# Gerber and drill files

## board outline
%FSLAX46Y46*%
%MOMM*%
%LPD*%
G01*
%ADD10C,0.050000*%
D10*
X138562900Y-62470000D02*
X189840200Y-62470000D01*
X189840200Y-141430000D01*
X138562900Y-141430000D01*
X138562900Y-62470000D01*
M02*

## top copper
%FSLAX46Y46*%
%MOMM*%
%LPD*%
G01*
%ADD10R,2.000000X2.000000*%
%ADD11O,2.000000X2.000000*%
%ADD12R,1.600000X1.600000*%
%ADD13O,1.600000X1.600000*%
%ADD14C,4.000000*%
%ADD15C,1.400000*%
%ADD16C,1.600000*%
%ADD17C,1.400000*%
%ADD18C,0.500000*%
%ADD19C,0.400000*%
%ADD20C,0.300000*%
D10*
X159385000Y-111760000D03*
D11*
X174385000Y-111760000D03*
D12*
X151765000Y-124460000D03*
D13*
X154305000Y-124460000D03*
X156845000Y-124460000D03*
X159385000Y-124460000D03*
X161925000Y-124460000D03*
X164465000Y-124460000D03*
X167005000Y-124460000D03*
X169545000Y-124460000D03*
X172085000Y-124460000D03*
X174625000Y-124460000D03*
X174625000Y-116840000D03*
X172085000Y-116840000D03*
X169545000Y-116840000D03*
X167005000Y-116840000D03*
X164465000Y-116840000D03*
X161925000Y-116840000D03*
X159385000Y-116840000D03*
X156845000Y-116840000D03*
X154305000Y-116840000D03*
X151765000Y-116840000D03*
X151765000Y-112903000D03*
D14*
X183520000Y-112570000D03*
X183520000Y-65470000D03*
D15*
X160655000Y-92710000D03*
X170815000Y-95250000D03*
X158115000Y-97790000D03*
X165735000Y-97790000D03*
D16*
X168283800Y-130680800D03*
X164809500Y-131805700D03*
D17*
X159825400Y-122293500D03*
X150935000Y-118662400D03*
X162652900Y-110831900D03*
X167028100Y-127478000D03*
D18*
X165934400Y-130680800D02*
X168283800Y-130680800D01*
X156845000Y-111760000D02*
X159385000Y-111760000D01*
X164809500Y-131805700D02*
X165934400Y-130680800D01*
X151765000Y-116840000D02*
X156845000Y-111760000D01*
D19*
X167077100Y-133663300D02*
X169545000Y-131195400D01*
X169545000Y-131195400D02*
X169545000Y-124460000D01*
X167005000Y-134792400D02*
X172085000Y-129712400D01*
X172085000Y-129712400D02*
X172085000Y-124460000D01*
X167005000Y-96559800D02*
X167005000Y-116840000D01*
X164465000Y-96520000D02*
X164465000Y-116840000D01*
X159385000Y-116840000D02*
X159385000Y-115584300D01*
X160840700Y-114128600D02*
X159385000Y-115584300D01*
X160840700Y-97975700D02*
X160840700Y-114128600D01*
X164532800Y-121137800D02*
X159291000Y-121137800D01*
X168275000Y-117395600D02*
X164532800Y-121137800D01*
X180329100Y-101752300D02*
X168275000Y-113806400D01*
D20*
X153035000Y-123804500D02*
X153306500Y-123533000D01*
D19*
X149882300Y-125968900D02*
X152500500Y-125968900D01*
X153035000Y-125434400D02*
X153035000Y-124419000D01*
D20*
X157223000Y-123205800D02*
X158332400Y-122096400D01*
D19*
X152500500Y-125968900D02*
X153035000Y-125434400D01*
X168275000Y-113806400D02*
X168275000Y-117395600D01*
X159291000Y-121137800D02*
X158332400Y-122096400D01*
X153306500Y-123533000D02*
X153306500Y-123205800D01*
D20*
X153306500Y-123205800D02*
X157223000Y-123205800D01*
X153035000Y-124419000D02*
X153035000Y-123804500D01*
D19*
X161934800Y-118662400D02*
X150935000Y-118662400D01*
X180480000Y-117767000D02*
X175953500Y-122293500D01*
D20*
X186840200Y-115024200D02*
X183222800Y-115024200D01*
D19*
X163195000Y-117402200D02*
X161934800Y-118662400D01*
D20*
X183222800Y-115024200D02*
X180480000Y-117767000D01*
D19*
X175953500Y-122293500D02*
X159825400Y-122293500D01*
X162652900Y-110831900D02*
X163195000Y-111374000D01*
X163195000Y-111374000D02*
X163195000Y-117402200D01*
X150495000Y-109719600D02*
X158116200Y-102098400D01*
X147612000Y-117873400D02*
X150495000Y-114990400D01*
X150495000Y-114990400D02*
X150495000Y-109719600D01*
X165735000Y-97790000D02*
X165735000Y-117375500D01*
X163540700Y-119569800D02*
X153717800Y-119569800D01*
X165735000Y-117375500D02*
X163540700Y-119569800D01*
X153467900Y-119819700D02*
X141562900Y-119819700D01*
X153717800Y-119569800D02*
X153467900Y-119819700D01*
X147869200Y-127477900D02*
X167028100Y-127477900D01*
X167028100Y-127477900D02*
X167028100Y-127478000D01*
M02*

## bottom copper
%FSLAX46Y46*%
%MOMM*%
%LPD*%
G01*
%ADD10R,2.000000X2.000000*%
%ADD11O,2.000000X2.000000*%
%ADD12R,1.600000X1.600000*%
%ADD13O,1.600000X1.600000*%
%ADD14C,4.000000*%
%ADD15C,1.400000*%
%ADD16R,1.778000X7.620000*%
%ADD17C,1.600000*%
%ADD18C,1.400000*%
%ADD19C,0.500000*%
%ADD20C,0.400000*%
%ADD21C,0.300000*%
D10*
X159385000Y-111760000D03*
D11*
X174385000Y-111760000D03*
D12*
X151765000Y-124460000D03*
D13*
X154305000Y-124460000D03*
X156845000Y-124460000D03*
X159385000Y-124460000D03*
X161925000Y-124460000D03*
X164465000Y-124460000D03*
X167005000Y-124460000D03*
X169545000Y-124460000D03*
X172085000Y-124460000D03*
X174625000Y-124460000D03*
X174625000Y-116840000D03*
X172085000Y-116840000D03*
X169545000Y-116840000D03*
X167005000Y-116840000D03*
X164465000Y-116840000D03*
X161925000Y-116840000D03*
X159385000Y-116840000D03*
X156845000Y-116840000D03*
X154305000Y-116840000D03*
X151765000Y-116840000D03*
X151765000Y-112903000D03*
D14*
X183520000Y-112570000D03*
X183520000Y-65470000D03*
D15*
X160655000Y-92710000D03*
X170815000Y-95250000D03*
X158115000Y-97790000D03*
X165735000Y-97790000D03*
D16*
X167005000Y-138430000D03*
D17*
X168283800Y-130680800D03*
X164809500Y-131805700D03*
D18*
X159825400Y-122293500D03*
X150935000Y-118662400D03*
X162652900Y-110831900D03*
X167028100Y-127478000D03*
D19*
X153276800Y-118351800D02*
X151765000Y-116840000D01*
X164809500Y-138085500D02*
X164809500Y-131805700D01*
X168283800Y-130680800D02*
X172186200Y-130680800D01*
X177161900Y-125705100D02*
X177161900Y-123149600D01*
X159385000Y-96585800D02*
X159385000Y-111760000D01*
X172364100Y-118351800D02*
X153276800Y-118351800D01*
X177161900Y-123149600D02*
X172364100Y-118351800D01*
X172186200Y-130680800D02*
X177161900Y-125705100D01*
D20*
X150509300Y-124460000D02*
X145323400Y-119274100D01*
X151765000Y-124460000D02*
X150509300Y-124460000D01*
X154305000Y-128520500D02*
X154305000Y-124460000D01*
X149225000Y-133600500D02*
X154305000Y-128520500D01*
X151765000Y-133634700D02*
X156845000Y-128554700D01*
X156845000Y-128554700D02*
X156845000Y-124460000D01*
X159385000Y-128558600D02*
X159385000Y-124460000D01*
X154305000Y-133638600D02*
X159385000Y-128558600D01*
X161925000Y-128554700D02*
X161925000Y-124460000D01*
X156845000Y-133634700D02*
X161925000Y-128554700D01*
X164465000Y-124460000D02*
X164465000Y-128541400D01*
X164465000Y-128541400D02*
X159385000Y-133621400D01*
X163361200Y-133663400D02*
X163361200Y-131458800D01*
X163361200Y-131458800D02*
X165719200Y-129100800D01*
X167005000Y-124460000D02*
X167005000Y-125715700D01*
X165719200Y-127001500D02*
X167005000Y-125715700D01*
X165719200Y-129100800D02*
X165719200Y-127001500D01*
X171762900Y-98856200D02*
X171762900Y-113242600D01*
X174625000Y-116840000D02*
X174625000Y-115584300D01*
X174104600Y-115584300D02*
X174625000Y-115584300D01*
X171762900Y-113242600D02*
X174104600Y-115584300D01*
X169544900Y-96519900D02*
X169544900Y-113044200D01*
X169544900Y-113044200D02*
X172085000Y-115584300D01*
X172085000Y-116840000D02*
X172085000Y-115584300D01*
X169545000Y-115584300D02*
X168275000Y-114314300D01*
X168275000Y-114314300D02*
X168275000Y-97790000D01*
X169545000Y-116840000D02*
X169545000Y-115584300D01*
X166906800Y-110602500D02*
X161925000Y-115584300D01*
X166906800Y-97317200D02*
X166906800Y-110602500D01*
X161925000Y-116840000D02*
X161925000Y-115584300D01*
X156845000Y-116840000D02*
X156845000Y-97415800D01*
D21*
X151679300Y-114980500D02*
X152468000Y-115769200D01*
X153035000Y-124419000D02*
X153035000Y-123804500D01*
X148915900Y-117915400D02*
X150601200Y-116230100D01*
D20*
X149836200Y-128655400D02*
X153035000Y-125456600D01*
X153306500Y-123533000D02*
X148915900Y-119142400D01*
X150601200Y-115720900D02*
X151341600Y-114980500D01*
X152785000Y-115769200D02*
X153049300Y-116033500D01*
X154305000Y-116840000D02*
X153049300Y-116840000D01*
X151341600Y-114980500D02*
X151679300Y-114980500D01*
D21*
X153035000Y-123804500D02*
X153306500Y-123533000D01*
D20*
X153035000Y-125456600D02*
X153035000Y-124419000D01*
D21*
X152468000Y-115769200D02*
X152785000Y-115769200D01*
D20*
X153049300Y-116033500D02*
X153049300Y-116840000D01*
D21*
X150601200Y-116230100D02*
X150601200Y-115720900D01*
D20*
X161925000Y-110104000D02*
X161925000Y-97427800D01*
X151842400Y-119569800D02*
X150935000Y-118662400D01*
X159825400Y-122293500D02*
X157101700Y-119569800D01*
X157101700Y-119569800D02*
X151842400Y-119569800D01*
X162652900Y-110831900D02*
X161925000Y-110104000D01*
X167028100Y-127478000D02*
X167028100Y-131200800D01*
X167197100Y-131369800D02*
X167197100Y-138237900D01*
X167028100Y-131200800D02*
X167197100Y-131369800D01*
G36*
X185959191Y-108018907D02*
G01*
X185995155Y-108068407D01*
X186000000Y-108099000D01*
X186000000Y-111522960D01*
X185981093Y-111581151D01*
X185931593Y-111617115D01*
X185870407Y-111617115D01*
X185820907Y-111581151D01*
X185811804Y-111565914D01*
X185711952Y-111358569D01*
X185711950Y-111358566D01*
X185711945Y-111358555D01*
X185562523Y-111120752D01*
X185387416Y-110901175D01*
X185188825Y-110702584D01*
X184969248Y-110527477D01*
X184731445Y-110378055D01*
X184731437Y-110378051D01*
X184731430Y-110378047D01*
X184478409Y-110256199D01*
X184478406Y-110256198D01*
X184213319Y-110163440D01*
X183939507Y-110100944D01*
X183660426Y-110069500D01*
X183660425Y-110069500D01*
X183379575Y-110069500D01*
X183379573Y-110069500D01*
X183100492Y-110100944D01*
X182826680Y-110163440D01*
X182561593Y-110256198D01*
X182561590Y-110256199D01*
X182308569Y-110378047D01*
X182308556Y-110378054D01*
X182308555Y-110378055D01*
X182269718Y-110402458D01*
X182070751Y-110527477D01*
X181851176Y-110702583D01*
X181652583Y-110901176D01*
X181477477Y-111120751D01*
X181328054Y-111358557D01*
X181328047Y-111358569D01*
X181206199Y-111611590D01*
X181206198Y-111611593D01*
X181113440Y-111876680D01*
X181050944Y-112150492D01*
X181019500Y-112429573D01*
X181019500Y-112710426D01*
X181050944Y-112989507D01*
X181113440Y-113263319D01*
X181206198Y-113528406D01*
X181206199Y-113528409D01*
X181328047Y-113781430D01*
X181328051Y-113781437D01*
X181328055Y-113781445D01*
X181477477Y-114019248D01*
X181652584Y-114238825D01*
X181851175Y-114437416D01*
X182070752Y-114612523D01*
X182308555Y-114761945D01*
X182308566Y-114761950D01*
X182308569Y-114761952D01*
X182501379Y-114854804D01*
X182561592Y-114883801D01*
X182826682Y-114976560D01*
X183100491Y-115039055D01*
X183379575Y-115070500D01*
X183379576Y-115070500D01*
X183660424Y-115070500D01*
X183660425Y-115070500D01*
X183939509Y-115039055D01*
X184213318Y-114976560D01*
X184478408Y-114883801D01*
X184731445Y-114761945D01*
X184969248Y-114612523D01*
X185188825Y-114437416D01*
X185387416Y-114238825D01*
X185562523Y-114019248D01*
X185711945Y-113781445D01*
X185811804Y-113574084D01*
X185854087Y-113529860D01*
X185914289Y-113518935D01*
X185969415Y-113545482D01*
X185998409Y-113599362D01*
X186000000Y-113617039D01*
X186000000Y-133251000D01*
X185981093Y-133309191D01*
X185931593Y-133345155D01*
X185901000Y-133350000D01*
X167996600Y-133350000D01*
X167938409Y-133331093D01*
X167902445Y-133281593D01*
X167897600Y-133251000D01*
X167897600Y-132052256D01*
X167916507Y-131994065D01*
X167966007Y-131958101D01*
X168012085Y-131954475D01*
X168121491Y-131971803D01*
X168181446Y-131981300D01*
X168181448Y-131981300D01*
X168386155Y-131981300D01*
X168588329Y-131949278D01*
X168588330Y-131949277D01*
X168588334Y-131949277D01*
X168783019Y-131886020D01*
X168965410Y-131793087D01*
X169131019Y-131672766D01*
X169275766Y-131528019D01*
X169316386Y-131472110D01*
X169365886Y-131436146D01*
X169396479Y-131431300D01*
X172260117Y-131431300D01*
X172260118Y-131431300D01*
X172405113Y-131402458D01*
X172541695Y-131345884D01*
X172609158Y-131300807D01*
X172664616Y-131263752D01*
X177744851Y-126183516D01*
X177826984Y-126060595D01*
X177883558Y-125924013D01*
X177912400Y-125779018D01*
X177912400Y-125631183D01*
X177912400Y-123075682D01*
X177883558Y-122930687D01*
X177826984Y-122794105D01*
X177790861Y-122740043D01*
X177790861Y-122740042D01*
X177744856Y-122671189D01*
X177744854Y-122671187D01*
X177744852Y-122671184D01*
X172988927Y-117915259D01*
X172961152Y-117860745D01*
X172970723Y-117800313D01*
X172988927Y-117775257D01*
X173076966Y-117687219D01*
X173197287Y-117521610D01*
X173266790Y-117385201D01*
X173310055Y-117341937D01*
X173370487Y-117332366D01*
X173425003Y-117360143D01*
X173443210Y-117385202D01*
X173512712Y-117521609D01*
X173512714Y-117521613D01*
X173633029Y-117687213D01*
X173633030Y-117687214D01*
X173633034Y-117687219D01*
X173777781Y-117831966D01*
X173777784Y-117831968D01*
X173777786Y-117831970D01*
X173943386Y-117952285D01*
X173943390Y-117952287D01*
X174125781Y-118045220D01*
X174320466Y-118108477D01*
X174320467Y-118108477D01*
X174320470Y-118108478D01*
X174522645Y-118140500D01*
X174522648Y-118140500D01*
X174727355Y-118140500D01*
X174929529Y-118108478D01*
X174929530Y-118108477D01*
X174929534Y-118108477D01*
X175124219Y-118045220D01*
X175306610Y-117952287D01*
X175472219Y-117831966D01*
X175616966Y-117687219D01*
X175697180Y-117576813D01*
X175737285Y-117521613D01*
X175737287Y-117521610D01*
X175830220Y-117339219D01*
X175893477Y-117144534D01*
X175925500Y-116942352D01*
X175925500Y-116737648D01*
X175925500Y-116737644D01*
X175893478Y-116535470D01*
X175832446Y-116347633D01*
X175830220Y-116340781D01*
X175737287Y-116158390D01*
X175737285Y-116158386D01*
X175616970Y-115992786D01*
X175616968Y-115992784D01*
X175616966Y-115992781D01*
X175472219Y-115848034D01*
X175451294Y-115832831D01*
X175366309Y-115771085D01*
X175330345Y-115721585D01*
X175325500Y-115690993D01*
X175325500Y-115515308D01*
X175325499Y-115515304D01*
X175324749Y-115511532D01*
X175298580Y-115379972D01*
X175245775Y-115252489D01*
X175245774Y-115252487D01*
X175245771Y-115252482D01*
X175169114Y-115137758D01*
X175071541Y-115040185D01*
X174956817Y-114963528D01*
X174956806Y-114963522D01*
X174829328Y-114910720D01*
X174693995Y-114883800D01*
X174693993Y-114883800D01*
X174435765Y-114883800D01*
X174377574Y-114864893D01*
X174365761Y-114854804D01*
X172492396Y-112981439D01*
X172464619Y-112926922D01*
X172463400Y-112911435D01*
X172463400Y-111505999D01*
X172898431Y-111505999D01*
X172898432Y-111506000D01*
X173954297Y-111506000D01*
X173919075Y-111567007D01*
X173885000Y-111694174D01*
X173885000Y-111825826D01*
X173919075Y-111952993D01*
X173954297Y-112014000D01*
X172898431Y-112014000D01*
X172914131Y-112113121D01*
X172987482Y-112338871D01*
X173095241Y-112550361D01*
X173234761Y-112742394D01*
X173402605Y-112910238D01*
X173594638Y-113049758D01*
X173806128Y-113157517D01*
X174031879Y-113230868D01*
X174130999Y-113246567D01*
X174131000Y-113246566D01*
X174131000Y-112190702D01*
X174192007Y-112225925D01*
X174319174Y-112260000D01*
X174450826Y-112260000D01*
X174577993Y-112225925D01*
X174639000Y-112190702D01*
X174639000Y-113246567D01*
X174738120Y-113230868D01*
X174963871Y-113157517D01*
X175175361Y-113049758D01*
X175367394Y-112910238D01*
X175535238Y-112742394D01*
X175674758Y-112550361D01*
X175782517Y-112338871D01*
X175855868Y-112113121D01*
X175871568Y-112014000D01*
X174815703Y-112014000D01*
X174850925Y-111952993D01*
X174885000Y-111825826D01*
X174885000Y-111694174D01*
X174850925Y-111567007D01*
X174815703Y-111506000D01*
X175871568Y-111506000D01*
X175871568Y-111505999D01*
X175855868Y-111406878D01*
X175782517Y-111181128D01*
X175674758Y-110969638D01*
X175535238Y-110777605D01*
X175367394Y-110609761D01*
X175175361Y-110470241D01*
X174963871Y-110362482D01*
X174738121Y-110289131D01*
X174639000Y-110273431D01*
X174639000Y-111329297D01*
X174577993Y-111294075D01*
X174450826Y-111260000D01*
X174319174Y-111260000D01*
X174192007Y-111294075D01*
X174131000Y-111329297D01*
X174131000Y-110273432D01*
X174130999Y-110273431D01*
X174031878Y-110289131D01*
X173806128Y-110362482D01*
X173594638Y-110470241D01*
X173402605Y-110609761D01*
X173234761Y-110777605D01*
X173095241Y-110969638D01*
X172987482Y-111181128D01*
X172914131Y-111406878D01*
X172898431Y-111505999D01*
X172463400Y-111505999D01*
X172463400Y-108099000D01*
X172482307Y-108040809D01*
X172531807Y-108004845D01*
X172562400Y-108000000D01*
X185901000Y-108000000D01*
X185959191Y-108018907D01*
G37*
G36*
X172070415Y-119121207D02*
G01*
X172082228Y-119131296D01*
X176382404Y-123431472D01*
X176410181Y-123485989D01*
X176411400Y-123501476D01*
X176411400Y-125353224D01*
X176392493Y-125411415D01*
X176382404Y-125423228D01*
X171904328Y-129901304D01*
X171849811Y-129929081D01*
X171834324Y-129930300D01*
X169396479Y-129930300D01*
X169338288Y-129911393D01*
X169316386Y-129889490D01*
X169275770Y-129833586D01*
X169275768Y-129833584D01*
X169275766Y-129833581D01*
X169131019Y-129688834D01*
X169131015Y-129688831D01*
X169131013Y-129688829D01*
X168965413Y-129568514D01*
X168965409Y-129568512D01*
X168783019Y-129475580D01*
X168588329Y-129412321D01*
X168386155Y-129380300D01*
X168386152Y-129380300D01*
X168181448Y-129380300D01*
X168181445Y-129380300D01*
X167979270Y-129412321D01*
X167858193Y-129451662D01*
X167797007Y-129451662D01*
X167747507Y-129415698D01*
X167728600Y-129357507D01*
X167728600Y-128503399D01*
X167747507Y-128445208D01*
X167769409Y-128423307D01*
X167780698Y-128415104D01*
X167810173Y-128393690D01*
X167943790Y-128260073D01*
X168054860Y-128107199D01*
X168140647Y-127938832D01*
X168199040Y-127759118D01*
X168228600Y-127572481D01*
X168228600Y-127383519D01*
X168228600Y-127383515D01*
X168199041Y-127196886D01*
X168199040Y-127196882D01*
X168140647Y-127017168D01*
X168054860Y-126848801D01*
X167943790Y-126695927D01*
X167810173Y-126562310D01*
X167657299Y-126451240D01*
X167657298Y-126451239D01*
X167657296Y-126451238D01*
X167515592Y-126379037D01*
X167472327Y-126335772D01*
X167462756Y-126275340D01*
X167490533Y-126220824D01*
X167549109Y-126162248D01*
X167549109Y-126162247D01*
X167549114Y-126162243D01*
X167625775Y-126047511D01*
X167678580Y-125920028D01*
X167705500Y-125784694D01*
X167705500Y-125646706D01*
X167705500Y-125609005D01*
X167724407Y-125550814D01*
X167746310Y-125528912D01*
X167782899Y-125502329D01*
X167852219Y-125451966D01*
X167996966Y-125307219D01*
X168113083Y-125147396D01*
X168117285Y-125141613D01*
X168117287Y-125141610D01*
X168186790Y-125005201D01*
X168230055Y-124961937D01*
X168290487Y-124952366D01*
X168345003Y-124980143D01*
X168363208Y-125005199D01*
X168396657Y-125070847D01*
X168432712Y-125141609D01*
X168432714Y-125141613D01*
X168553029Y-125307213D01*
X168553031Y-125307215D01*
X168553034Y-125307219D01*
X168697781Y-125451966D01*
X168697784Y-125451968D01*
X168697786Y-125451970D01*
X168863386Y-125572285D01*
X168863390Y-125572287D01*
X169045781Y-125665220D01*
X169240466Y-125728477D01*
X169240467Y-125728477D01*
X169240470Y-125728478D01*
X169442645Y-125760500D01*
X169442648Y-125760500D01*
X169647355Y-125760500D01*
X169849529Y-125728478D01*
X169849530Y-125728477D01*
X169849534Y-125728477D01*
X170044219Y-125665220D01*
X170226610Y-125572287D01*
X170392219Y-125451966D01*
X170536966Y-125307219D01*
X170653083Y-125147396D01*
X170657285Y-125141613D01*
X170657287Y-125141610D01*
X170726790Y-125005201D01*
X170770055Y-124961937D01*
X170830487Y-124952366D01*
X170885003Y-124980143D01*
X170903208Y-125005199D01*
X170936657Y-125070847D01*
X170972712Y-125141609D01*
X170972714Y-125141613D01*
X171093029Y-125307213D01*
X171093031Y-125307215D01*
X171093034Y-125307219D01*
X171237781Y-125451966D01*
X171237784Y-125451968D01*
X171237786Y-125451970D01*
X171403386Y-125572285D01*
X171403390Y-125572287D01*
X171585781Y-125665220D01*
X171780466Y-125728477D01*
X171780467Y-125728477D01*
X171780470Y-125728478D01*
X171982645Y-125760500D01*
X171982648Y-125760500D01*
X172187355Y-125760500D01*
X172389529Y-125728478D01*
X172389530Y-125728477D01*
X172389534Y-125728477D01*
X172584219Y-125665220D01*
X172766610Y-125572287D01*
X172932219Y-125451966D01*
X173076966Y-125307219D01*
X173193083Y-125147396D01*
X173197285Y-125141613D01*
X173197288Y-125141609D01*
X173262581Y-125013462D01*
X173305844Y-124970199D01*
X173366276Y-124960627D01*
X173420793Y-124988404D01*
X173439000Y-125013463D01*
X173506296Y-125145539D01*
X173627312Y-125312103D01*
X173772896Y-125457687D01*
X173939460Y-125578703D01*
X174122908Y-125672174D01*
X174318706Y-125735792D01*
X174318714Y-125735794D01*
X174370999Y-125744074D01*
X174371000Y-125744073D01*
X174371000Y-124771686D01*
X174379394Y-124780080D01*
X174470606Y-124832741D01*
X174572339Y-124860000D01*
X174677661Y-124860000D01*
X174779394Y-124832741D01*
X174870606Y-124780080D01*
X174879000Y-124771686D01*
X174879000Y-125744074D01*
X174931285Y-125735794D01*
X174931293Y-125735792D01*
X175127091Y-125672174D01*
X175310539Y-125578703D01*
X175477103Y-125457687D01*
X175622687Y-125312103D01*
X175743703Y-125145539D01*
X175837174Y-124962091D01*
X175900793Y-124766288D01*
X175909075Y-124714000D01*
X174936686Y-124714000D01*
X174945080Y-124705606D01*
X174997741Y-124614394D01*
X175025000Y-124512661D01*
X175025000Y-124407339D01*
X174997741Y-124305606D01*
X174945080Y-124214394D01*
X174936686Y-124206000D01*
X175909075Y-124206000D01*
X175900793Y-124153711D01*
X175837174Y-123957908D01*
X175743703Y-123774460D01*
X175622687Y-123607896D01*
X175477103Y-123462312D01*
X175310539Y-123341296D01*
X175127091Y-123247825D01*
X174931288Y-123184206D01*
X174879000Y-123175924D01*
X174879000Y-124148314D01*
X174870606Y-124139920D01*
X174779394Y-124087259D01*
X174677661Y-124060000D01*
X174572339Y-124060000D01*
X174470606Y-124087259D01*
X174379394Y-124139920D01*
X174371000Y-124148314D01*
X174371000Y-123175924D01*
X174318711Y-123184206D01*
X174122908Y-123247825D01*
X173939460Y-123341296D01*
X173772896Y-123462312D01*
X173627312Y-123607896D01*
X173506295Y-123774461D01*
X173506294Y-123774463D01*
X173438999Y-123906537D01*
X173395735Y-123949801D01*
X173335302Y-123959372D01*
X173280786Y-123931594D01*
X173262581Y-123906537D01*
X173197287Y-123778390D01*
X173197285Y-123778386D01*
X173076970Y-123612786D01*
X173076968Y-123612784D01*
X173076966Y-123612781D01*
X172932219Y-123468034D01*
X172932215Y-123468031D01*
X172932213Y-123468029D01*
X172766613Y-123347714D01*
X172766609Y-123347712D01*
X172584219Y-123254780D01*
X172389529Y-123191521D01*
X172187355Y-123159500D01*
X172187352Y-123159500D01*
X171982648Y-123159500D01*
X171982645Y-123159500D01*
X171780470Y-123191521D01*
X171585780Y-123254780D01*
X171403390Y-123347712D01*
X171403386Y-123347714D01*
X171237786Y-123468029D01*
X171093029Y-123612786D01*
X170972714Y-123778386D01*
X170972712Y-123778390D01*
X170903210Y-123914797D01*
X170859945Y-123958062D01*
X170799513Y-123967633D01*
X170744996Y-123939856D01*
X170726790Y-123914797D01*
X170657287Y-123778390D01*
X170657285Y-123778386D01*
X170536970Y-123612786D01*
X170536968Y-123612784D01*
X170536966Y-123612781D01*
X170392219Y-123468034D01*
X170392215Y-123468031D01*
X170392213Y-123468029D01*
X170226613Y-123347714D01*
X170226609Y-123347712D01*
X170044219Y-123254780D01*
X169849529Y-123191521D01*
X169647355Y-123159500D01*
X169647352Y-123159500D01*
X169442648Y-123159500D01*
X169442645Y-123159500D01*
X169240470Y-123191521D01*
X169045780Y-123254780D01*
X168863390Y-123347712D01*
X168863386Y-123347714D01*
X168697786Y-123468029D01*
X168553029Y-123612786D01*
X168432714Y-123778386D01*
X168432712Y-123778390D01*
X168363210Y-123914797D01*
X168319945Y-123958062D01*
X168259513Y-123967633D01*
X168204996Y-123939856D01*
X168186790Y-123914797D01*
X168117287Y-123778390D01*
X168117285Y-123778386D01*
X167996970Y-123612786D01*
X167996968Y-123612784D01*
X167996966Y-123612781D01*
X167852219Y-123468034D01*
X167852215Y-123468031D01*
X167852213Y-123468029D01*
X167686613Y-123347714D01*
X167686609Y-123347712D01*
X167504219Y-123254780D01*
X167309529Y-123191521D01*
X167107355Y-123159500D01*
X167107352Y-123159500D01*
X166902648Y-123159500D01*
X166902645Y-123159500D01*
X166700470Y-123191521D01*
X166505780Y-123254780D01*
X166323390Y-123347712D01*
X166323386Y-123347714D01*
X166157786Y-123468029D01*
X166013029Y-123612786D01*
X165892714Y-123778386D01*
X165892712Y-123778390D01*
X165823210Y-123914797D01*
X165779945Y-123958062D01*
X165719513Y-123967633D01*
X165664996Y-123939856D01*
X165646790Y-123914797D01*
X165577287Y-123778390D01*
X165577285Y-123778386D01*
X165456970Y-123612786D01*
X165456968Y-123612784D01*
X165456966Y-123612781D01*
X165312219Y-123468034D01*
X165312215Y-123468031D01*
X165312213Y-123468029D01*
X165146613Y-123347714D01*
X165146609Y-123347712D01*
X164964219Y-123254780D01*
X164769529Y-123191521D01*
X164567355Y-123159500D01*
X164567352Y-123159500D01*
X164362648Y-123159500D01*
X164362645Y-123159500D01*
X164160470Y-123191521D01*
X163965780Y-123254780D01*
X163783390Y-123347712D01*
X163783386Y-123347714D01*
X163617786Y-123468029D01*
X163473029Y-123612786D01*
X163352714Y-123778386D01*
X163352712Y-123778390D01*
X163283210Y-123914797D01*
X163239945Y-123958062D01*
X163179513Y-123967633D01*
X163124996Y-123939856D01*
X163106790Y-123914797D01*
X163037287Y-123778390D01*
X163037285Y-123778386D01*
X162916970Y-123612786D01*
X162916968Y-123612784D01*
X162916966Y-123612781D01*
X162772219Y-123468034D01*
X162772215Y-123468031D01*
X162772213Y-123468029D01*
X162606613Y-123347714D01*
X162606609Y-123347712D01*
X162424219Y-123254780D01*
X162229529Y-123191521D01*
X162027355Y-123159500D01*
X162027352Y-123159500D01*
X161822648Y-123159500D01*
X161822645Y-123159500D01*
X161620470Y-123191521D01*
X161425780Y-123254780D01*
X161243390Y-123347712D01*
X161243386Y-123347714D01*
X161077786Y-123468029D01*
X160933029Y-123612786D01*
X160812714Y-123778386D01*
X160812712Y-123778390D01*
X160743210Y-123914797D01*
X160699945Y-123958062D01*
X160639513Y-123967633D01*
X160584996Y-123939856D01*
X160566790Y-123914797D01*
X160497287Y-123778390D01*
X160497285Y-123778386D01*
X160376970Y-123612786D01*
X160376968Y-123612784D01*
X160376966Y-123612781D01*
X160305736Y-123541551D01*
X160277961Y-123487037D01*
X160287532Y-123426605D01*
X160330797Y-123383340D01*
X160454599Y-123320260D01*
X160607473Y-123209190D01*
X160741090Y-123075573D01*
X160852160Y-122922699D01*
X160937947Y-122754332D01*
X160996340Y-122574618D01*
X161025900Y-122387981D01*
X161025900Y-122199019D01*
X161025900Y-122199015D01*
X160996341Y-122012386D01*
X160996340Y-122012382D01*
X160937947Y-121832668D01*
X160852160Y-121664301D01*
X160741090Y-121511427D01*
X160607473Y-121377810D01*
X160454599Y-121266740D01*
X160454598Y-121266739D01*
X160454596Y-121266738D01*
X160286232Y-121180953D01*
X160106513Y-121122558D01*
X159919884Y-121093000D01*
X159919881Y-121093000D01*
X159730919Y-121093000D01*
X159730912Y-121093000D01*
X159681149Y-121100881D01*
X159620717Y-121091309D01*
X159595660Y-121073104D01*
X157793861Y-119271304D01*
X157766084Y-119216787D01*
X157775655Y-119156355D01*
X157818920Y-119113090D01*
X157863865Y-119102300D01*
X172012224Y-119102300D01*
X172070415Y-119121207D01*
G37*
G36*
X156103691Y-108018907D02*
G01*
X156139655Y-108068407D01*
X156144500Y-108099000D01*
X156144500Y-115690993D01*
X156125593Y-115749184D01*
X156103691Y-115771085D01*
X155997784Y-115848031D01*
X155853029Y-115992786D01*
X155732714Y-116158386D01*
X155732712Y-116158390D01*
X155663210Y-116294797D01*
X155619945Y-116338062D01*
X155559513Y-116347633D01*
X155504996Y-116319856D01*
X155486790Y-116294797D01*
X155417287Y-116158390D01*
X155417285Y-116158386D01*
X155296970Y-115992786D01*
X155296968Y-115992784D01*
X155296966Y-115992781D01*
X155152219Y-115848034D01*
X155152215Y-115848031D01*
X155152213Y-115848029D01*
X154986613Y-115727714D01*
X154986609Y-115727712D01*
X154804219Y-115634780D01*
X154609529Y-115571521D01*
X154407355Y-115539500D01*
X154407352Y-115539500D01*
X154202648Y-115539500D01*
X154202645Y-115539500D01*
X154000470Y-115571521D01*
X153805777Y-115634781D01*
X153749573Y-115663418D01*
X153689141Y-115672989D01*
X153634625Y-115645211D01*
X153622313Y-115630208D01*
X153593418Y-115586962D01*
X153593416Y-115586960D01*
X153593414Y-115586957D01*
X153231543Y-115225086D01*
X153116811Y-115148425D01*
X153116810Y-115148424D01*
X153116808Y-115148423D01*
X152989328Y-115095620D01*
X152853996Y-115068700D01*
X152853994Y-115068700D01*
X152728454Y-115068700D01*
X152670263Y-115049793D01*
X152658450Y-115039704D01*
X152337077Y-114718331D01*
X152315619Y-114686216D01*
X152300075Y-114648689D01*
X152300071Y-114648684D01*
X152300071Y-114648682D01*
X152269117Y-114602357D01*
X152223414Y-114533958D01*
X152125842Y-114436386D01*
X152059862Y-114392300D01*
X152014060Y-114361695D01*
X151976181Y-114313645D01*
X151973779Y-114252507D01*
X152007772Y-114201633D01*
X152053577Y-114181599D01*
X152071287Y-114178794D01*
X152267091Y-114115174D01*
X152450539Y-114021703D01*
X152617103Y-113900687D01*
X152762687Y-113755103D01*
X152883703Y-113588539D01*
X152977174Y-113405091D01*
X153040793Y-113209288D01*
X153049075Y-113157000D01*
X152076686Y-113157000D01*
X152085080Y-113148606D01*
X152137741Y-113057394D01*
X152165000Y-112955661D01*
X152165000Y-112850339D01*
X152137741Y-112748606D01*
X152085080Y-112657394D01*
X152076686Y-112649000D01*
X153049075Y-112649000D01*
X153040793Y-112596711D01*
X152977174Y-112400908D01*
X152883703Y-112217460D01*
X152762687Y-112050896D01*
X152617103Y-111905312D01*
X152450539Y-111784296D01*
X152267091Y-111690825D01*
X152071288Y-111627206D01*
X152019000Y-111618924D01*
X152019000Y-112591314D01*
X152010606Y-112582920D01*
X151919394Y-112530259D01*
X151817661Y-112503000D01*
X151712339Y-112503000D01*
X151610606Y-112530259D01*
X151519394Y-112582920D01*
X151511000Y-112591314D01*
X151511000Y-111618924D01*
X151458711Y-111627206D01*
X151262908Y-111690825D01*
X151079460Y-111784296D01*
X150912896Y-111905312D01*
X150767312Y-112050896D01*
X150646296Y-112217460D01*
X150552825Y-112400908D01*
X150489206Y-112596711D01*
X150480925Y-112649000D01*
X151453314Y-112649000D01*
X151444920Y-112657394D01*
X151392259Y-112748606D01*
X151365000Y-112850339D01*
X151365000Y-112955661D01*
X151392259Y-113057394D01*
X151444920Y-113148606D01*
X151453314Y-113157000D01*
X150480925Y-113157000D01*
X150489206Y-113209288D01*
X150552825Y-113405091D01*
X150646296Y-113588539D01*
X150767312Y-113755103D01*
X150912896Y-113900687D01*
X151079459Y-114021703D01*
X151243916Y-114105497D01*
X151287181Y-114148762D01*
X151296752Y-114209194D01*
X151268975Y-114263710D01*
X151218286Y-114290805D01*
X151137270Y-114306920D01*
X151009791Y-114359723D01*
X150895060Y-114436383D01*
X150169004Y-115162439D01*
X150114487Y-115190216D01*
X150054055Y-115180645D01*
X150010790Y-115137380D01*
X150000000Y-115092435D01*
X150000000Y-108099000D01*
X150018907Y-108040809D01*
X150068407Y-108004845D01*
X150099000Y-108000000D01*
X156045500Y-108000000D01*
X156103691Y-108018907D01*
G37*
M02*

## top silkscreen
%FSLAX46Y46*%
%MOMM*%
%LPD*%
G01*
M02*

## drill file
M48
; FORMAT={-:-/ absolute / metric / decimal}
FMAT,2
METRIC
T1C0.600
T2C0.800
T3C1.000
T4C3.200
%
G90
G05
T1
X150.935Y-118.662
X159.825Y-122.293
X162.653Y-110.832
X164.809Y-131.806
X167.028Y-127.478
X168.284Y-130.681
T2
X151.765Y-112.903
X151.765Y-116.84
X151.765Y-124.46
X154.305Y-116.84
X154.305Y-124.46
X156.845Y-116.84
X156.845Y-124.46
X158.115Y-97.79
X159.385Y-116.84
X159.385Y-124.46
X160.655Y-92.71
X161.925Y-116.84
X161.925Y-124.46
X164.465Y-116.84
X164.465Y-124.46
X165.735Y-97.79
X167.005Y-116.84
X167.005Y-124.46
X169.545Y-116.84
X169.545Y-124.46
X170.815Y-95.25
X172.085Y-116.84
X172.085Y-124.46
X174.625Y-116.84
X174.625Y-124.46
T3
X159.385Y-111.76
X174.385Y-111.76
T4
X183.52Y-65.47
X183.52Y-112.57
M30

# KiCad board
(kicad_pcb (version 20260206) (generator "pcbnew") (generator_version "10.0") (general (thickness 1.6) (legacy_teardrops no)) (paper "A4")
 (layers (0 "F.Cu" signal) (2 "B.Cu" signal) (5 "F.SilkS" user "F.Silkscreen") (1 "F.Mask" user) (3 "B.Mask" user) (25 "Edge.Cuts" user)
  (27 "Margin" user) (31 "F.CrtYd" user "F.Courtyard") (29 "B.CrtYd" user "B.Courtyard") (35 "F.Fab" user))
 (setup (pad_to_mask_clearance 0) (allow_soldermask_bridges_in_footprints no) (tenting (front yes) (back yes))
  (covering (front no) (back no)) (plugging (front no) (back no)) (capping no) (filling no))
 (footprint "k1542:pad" (layer "F.Cu") (at 159.385 111.76)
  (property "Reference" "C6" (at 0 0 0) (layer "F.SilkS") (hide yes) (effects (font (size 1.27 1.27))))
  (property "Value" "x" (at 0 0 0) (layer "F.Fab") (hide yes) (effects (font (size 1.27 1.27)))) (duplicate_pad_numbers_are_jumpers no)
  (pad "1" thru_hole rect (at 0 0) (size 2 2) (drill 1) (layers "*.Cu" "*.Mask") (remove_unused_layers no) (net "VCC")))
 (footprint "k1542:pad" (layer "F.Cu") (at 174.385 111.76)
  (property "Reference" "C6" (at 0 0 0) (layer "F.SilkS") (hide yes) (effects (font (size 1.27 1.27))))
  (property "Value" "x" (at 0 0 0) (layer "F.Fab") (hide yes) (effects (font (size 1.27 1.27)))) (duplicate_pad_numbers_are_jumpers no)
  (pad "2" thru_hole oval (at 0 0) (size 2 2) (drill 1) (layers "*.Cu" "*.Mask") (remove_unused_layers no) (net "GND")))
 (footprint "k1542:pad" (layer "F.Cu") (at 151.765 124.46 90)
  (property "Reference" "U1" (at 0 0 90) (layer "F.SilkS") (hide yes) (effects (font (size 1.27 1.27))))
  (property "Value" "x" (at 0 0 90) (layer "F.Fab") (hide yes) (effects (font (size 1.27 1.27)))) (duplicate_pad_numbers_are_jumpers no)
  (pad "1" thru_hole rect (at 0 0 90) (size 1.6 1.6) (drill 0.8) (layers "*.Cu" "*.Mask") (remove_unused_layers no) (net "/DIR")))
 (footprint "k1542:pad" (layer "F.Cu") (at 154.305 124.46 90)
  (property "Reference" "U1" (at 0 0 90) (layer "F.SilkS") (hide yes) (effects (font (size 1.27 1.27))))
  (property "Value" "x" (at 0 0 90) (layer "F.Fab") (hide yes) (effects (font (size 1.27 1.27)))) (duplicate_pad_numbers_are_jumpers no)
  (pad "2" thru_hole oval (at 0 0 90) (size 1.6 1.6) (drill 0.8) (layers "*.Cu" "*.Mask") (remove_unused_layers no) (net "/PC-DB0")))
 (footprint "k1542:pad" (layer "F.Cu") (at 156.845 124.46 90)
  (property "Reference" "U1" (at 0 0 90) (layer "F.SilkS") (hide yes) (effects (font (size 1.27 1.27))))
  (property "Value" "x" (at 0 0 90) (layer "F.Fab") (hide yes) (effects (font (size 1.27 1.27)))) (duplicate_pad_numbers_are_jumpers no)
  (pad "3" thru_hole oval (at 0 0 90) (size 1.6 1.6) (drill 0.8) (layers "*.Cu" "*.Mask") (remove_unused_layers no) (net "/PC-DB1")))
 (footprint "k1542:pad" (layer "F.Cu") (at 159.385 124.46 90)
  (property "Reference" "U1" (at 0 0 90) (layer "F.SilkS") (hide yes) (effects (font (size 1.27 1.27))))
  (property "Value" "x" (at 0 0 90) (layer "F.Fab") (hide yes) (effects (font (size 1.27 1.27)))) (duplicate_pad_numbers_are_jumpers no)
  (pad "4" thru_hole oval (at 0 0 90) (size 1.6 1.6) (drill 0.8) (layers "*.Cu" "*.Mask") (remove_unused_layers no) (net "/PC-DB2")))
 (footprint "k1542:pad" (layer "F.Cu") (at 161.925 124.46 90)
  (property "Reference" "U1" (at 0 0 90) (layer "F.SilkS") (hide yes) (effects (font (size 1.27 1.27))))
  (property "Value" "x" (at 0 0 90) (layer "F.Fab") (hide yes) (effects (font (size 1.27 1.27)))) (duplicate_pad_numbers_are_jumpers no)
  (pad "5" thru_hole oval (at 0 0 90) (size 1.6 1.6) (drill 0.8) (layers "*.Cu" "*.Mask") (remove_unused_layers no) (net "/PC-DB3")))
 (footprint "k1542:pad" (layer "F.Cu") (at 164.465 124.46 90)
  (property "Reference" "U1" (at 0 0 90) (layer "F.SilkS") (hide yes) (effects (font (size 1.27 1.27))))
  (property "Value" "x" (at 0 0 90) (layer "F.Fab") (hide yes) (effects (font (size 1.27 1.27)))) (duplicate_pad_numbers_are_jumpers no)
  (pad "6" thru_hole oval (at 0 0 90) (size 1.6 1.6) (drill 0.8) (layers "*.Cu" "*.Mask") (remove_unused_layers no) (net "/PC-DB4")))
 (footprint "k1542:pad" (layer "F.Cu") (at 167.005 124.46 90)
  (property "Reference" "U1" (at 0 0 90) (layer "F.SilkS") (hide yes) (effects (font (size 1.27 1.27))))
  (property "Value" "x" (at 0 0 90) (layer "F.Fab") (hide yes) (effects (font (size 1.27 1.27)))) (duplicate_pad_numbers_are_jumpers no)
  (pad "7" thru_hole oval (at 0 0 90) (size 1.6 1.6) (drill 0.8) (layers "*.Cu" "*.Mask") (remove_unused_layers no) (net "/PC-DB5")))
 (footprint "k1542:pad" (layer "F.Cu") (at 169.545 124.46 90)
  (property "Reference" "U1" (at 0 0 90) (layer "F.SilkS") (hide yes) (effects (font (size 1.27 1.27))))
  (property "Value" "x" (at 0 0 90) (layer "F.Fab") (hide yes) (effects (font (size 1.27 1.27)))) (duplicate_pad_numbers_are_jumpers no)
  (pad "8" thru_hole oval (at 0 0 90) (size 1.6 1.6) (drill 0.8) (layers "*.Cu" "*.Mask") (remove_unused_layers no) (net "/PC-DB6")))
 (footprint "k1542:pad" (layer "F.Cu") (at 172.085 124.46 90)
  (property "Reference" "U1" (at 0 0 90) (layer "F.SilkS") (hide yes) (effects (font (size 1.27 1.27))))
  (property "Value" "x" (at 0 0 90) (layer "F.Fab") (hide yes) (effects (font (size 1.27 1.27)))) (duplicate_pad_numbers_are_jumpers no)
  (pad "9" thru_hole oval (at 0 0 90) (size 1.6 1.6) (drill 0.8) (layers "*.Cu" "*.Mask") (remove_unused_layers no) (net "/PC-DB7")))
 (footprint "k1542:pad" (layer "F.Cu") (at 174.625 124.46 90)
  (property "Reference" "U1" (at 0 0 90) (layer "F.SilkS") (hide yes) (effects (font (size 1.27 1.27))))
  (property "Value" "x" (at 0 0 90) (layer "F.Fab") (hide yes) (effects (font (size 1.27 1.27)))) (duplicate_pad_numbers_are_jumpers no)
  (pad "10" thru_hole oval (at 0 0 90) (size 1.6 1.6) (drill 0.8) (layers "*.Cu" "*.Mask") (remove_unused_layers no) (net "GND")))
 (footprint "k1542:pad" (layer "F.Cu") (at 174.625 116.84 90)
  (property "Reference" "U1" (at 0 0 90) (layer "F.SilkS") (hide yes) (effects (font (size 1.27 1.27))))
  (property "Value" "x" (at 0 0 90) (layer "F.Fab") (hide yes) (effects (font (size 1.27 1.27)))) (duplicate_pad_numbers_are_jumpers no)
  (pad "11" thru_hole oval (at 0 0 90) (size 1.6 1.6) (drill 0.8) (layers "*.Cu" "*.Mask") (remove_unused_layers no) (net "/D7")))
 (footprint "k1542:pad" (layer "F.Cu") (at 172.085 116.84 90)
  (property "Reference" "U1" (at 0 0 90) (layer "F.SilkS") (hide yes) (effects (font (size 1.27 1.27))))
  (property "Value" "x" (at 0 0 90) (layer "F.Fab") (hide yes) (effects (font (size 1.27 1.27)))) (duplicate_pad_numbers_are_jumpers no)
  (pad "12" thru_hole oval (at 0 0 90) (size 1.6 1.6) (drill 0.8) (layers "*.Cu" "*.Mask") (remove_unused_layers no) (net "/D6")))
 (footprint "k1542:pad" (layer "F.Cu") (at 169.545 116.84 90)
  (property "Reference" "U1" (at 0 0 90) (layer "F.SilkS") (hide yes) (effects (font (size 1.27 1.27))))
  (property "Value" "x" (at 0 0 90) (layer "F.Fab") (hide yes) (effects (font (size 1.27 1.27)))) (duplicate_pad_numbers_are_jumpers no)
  (pad "13" thru_hole oval (at 0 0 90) (size 1.6 1.6) (drill 0.8) (layers "*.Cu" "*.Mask") (remove_unused_layers no) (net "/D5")))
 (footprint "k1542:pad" (layer "F.Cu") (at 167.005 116.84 90)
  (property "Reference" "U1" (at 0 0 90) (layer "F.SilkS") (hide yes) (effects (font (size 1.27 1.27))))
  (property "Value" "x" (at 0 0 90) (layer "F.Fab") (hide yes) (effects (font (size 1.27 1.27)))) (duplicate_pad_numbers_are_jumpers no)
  (pad "14" thru_hole oval (at 0 0 90) (size 1.6 1.6) (drill 0.8) (layers "*.Cu" "*.Mask") (remove_unused_layers no) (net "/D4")))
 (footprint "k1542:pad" (layer "F.Cu") (at 164.465 116.84 90)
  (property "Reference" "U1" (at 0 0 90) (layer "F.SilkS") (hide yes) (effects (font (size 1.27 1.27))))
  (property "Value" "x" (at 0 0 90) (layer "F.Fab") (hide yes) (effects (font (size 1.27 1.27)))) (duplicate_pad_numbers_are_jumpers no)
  (pad "15" thru_hole oval (at 0 0 90) (size 1.6 1.6) (drill 0.8) (layers "*.Cu" "*.Mask") (remove_unused_layers no) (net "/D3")))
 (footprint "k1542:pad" (layer "F.Cu") (at 161.925 116.84 90)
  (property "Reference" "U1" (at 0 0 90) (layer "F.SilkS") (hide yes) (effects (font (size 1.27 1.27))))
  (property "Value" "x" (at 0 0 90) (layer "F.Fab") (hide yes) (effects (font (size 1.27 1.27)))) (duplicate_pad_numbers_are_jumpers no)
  (pad "16" thru_hole oval (at 0 0 90) (size 1.6 1.6) (drill 0.8) (layers "*.Cu" "*.Mask") (remove_unused_layers no) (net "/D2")))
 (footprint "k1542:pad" (layer "F.Cu") (at 159.385 116.84 90)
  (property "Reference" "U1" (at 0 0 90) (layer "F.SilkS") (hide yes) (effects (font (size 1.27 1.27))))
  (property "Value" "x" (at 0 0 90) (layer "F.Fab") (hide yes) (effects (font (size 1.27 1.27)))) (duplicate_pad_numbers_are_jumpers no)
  (pad "17" thru_hole oval (at 0 0 90) (size 1.6 1.6) (drill 0.8) (layers "*.Cu" "*.Mask") (remove_unused_layers no) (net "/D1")))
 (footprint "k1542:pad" (layer "F.Cu") (at 156.845 116.84 90)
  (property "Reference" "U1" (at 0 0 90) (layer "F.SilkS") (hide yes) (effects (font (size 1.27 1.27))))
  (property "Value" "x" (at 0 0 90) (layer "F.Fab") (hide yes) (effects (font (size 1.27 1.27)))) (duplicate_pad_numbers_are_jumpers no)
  (pad "18" thru_hole oval (at 0 0 90) (size 1.6 1.6) (drill 0.8) (layers "*.Cu" "*.Mask") (remove_unused_layers no) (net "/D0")))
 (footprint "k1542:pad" (layer "F.Cu") (at 154.305 116.84 90)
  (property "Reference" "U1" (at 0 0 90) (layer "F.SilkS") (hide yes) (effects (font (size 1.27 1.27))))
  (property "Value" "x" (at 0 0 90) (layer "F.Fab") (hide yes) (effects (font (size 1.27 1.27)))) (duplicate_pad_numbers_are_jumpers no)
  (pad "19" thru_hole oval (at 0 0 90) (size 1.6 1.6) (drill 0.8) (layers "*.Cu" "*.Mask") (remove_unused_layers no) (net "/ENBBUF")))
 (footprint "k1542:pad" (layer "F.Cu") (at 151.765 116.84 90)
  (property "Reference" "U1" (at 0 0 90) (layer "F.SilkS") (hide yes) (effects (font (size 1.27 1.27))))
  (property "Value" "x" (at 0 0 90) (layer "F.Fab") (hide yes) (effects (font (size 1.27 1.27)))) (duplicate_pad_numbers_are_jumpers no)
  (pad "20" thru_hole oval (at 0 0 90) (size 1.6 1.6) (drill 0.8) (layers "*.Cu" "*.Mask") (remove_unused_layers no) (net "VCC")))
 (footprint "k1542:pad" (layer "F.Cu") (at 151.765 112.903 90)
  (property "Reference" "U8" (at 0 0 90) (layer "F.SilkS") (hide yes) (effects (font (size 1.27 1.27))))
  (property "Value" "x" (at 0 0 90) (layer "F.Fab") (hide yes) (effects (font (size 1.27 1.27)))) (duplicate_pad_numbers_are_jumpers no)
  (pad "12" thru_hole oval (at 0 0 90) (size 1.6 1.6) (drill 0.8) (layers "*.Cu" "*.Mask") (remove_unused_layers no) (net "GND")))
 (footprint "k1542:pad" (layer "F.Cu") (at 183.52 112.57 90)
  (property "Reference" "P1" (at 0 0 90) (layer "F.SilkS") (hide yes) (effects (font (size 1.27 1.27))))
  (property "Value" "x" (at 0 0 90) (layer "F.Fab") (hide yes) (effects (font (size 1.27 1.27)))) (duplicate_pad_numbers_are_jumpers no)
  (pad "0" thru_hole circle (at 0 0 90) (size 4 4) (drill 3.2) (layers "*.Cu" "*.Mask") (remove_unused_layers no)))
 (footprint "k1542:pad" (layer "F.Cu") (at 183.52 65.47 90)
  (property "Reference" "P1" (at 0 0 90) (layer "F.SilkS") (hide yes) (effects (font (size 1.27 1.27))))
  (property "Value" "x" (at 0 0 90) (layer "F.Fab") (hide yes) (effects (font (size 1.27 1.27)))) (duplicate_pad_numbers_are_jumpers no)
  (pad "0" thru_hole circle (at 0 0 90) (size 4 4) (drill 3.2) (layers "*.Cu" "*.Mask") (remove_unused_layers no)))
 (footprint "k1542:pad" (layer "F.Cu") (at 160.655 92.71 180)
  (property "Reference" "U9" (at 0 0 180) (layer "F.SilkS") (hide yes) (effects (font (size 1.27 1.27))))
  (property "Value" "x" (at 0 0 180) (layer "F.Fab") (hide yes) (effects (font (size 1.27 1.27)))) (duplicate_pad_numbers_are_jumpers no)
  (pad "L8" thru_hole circle (at 0 0 180) (size 1.4 1.4) (drill 0.8) (layers "*.Cu" "*.Mask") (remove_unused_layers no) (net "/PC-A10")))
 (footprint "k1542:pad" (layer "F.Cu") (at 170.815 95.25 180)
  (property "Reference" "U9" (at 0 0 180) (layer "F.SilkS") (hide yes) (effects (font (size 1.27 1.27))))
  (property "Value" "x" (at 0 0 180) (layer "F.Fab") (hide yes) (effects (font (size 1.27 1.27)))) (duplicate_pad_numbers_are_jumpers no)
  (pad "M12" thru_hole circle (at 0 0 180) (size 1.4 1.4) (drill 0.8) (layers "*.Cu" "*.Mask") (remove_unused_layers no) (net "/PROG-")))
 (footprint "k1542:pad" (layer "F.Cu") (at 158.115 97.79 180)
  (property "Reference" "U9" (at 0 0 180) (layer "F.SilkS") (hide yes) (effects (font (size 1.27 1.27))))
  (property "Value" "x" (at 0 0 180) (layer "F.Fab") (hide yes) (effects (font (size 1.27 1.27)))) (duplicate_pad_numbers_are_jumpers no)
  (pad "N7" thru_hole circle (at 0 0 180) (size 1.4 1.4) (drill 0.8) (layers "*.Cu" "*.Mask") (remove_unused_layers no) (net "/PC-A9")))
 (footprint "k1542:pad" (layer "F.Cu") (at 165.735 97.79 180)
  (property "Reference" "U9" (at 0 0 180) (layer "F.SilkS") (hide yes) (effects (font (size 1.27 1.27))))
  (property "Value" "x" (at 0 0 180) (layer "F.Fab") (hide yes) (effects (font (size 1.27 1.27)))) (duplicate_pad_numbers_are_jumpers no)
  (pad "N10" thru_hole circle (at 0 0 180) (size 1.4 1.4) (drill 0.8) (layers "*.Cu" "*.Mask") (remove_unused_layers no) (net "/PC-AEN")))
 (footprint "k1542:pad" (layer "F.Cu") (at 167.005 138.43)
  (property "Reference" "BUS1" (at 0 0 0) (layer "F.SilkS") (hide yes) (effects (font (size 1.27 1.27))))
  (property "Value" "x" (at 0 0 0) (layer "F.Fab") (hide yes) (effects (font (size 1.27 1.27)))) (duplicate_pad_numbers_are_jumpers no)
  (pad "2" smd rect (at 0 0) (size 1.778 7.62) (layers "B.Cu" "B.Mask") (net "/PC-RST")))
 (gr_rect (start 138.5629 62.47) (end 189.8402 141.43) (stroke (width 0.05) (type default)) (fill no) (layer "Edge.Cuts"))
 (segment (start 165.9344 130.6808) (end 168.2838 130.6808) (width 0.5) (locked yes) (layer "F.Cu") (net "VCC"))
 (segment (start 156.845 111.76) (end 159.385 111.76) (width 0.5) (locked yes) (layer "F.Cu") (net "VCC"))
 (segment (start 164.8095 131.8057) (end 165.9344 130.6808) (width 0.5) (locked yes) (layer "F.Cu") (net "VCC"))
 (segment (start 151.765 116.84) (end 156.845 111.76) (width 0.5) (locked yes) (layer "F.Cu") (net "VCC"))
 (via (at 168.2838 130.6808) (size 1.6) (drill 0.6) (layers "F.Cu" "B.Cu") (locked yes) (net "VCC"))
 (via (at 164.8095 131.8057) (size 1.6) (drill 0.6) (layers "F.Cu" "B.Cu") (locked yes) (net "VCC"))
 (segment (start 153.2768 118.3518) (end 151.765 116.84) (width 0.5) (locked yes) (layer "B.Cu") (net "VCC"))
 (segment (start 164.8095 138.0855) (end 164.8095 131.8057) (width 0.5) (locked yes) (layer "B.Cu") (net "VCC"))
 (segment (start 168.2838 130.6808) (end 172.1862 130.6808) (width 0.5) (locked yes) (layer "B.Cu") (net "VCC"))
 (segment (start 177.1619 125.7051) (end 177.1619 123.1496) (width 0.5) (locked yes) (layer "B.Cu") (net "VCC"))
 (segment (start 159.385 96.5858) (end 159.385 111.76) (width 0.5) (locked yes) (layer "B.Cu") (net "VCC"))
 (segment (start 172.3641 118.3518) (end 153.2768 118.3518) (width 0.5) (locked yes) (layer "B.Cu") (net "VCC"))
 (segment (start 177.1619 123.1496) (end 172.3641 118.3518) (width 0.5) (locked yes) (layer "B.Cu") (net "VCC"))
 (segment (start 172.1862 130.6808) (end 177.1619 125.7051) (width 0.5) (locked yes) (layer "B.Cu") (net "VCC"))
 (segment (start 150.5093 124.46) (end 145.3234 119.2741) (width 0.4) (locked yes) (layer "B.Cu") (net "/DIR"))
 (segment (start 151.765 124.46) (end 150.5093 124.46) (width 0.4) (locked yes) (layer "B.Cu") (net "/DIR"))
 (segment (start 154.305 128.5205) (end 154.305 124.46) (width 0.4) (locked yes) (layer "B.Cu") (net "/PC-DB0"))
 (segment (start 149.225 133.6005) (end 154.305 128.5205) (width 0.4) (locked yes) (layer "B.Cu") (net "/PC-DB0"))
 (segment (start 151.765 133.6347) (end 156.845 128.5547) (width 0.4) (locked yes) (layer "B.Cu") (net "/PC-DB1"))
 (segment (start 156.845 128.5547) (end 156.845 124.46) (width 0.4) (locked yes) (layer "B.Cu") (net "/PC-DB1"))
 (segment (start 159.385 128.5586) (end 159.385 124.46) (width 0.4) (locked yes) (layer "B.Cu") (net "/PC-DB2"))
 (segment (start 154.305 133.6386) (end 159.385 128.5586) (width 0.4) (locked yes) (layer "B.Cu") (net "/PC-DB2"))
 (segment (start 161.925 128.5547) (end 161.925 124.46) (width 0.4) (locked yes) (layer "B.Cu") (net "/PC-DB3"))
 (segment (start 156.845 133.6347) (end 161.925 128.5547) (width 0.4) (locked yes) (layer "B.Cu") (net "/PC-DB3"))
 (segment (start 164.465 124.46) (end 164.465 128.5414) (width 0.4) (locked yes) (layer "B.Cu") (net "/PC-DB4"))
 (segment (start 164.465 128.5414) (end 159.385 133.6214) (width 0.4) (locked yes) (layer "B.Cu") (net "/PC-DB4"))
 (segment (start 163.3612 133.6634) (end 163.3612 131.4588) (width 0.4) (locked yes) (layer "B.Cu") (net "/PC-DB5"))
 (segment (start 163.3612 131.4588) (end 165.7192 129.1008) (width 0.4) (locked yes) (layer "B.Cu") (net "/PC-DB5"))
 (segment (start 167.005 124.46) (end 167.005 125.7157) (width 0.4) (locked yes) (layer "B.Cu") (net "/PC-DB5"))
 (segment (start 165.7192 127.0015) (end 167.005 125.7157) (width 0.4) (locked yes) (layer "B.Cu") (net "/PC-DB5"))
 (segment (start 165.7192 129.1008) (end 165.7192 127.0015) (width 0.4) (locked yes) (layer "B.Cu") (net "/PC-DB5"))
 (segment (start 167.0771 133.6633) (end 169.545 131.1954) (width 0.4) (locked yes) (layer "F.Cu") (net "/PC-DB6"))
 (segment (start 169.545 131.1954) (end 169.545 124.46) (width 0.4) (locked yes) (layer "F.Cu") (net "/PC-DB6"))
 (segment (start 167.005 134.7924) (end 172.085 129.7124) (width 0.4) (locked yes) (layer "F.Cu") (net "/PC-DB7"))
 (segment (start 172.085 129.7124) (end 172.085 124.46) (width 0.4) (locked yes) (layer "F.Cu") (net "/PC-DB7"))
 (segment (start 171.7629 98.8562) (end 171.7629 113.2426) (width 0.4) (locked yes) (layer "B.Cu") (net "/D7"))
 (segment (start 174.625 116.84) (end 174.625 115.5843) (width 0.4) (locked yes) (layer "B.Cu") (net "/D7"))
 (segment (start 174.1046 115.5843) (end 174.625 115.5843) (width 0.4) (locked yes) (layer "B.Cu") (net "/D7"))
 (segment (start 171.7629 113.2426) (end 174.1046 115.5843) (width 0.4) (locked yes) (layer "B.Cu") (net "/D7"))
 (segment (start 169.5449 96.5199) (end 169.5449 113.0442) (width 0.4) (locked yes) (layer "B.Cu") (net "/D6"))
 (segment (start 169.5449 113.0442) (end 172.085 115.5843) (width 0.4) (locked yes) (layer "B.Cu") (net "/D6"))
 (segment (start 172.085 116.84) (end 172.085 115.5843) (width 0.4) (locked yes) (layer "B.Cu") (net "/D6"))
 (segment (start 169.545 115.5843) (end 168.275 114.3143) (width 0.4) (locked yes) (layer "B.Cu") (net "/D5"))
 (segment (start 168.275 114.3143) (end 168.275 97.79) (width 0.4) (locked yes) (layer "B.Cu") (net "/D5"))
 (segment (start 169.545 116.84) (end 169.545 115.5843) (width 0.4) (locked yes) (layer "B.Cu") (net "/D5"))
 (segment (start 167.005 96.5598) (end 167.005 116.84) (width 0.4) (locked yes) (layer "F.Cu") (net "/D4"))
 (segment (start 164.465 96.52) (end 164.465 116.84) (width 0.4) (locked yes) (layer "F.Cu") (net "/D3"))
 (segment (start 166.9068 110.6025) (end 161.925 115.5843) (width 0.4) (locked yes) (layer "B.Cu") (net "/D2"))
 (segment (start 166.9068 97.3172) (end 166.9068 110.6025) (width 0.4) (locked yes) (layer "B.Cu") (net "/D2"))
 (segment (start 161.925 116.84) (end 161.925 115.5843) (width 0.4) (locked yes) (layer "B.Cu") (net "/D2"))
 (segment (start 159.385 116.84) (end 159.385 115.5843) (width 0.4) (locked yes) (layer "F.Cu") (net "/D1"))
 (segment (start 160.8407 114.1286) (end 159.385 115.5843) (width 0.4) (locked yes) (layer "F.Cu") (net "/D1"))
 (segment (start 160.8407 97.9757) (end 160.8407 114.1286) (width 0.4) (locked yes) (layer "F.Cu") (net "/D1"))
 (segment (start 156.845 116.84) (end 156.845 97.4158) (width 0.4) (locked yes) (layer "B.Cu") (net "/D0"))
 (segment (start 151.6793 114.9805) (end 152.468 115.7692) (width 0.3) (locked yes) (layer "B.Cu") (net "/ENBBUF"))
 (segment (start 153.035 124.419) (end 153.035 123.8045) (width 0.3) (locked yes) (layer "B.Cu") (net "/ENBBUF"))
 (segment (start 148.9159 117.9154) (end 150.6012 116.2301) (width 0.3) (locked yes) (layer "B.Cu") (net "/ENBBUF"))
 (segment (start 149.8362 128.6554) (end 153.035 125.4566) (width 0.4) (locked yes) (layer "B.Cu") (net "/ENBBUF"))
 (segment (start 153.3065 123.533) (end 148.9159 119.1424) (width 0.4) (locked yes) (layer "B.Cu") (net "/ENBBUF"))
 (segment (start 150.6012 115.7209) (end 151.3416 114.9805) (width 0.4) (locked yes) (layer "B.Cu") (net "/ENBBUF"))
 (segment (start 152.785 115.7692) (end 153.0493 116.0335) (width 0.4) (locked yes) (layer "B.Cu") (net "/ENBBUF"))
 (segment (start 154.305 116.84) (end 153.0493 116.84) (width 0.4) (locked yes) (layer "B.Cu") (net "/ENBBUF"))
 (segment (start 151.3416 114.9805) (end 151.6793 114.9805) (width 0.4) (locked yes) (layer "B.Cu") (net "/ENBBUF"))
 (segment (start 153.035 123.8045) (end 153.3065 123.533) (width 0.3) (locked yes) (layer "B.Cu") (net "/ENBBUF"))
 (segment (start 153.035 125.4566) (end 153.035 124.419) (width 0.4) (locked yes) (layer "B.Cu") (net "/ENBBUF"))
 (segment (start 152.468 115.7692) (end 152.785 115.7692) (width 0.3) (locked yes) (layer "B.Cu") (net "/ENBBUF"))
 (segment (start 153.0493 116.0335) (end 153.0493 116.84) (width 0.4) (locked yes) (layer "B.Cu") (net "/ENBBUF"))
 (segment (start 150.6012 116.2301) (end 150.6012 115.7209) (width 0.3) (locked yes) (layer "B.Cu") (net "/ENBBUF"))
 (segment (start 164.5328 121.1378) (end 159.291 121.1378) (width 0.4) (locked yes) (layer "F.Cu") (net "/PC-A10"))
 (segment (start 168.275 117.3956) (end 164.5328 121.1378) (width 0.4) (locked yes) (layer "F.Cu") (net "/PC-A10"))
 (segment (start 180.3291 101.7523) (end 168.275 113.8064) (width 0.4) (locked yes) (layer "F.Cu") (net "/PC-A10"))
 (segment (start 153.035 123.8045) (end 153.3065 123.533) (width 0.3) (locked yes) (layer "F.Cu") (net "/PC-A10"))
 (segment (start 149.8823 125.9689) (end 152.5005 125.9689) (width 0.4) (locked yes) (layer "F.Cu") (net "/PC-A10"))
 (segment (start 153.035 125.4344) (end 153.035 124.419) (width 0.4) (locked yes) (layer "F.Cu") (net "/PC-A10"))
 (segment (start 157.223 123.2058) (end 158.3324 122.0964) (width 0.3) (locked yes) (layer "F.Cu") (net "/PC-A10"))
 (segment (start 152.5005 125.9689) (end 153.035 125.4344) (width 0.4) (locked yes) (layer "F.Cu") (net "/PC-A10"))
 (segment (start 168.275 113.8064) (end 168.275 117.3956) (width 0.4) (locked yes) (layer "F.Cu") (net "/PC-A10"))
 (segment (start 159.291 121.1378) (end 158.3324 122.0964) (width 0.4) (locked yes) (layer "F.Cu") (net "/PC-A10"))
 (segment (start 153.3065 123.533) (end 153.3065 123.2058) (width 0.4) (locked yes) (layer "F.Cu") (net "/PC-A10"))
 (segment (start 153.3065 123.2058) (end 157.223 123.2058) (width 0.3) (locked yes) (layer "F.Cu") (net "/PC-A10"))
 (segment (start 153.035 124.419) (end 153.035 123.8045) (width 0.3) (locked yes) (layer "F.Cu") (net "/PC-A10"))
 (segment (start 161.9348 118.6624) (end 150.935 118.6624) (width 0.4) (locked yes) (layer "F.Cu") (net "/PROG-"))
 (segment (start 180.48 117.767) (end 175.9535 122.2935) (width 0.4) (locked yes) (layer "F.Cu") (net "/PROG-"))
 (segment (start 186.8402 115.0242) (end 183.2228 115.0242) (width 0.3) (locked yes) (layer "F.Cu") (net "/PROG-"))
 (segment (start 163.195 117.4022) (end 161.9348 118.6624) (width 0.4) (locked yes) (layer "F.Cu") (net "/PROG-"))
 (segment (start 183.2228 115.0242) (end 180.48 117.767) (width 0.3) (locked yes) (layer "F.Cu") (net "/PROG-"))
 (segment (start 175.9535 122.2935) (end 159.8254 122.2935) (width 0.4) (locked yes) (layer "F.Cu") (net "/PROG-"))
 (segment (start 162.6529 110.8319) (end 163.195 111.374) (width 0.4) (locked yes) (layer "F.Cu") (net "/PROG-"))
 (segment (start 163.195 111.374) (end 163.195 117.4022) (width 0.4) (locked yes) (layer "F.Cu") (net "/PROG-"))
 (via (at 159.8254 122.2935) (size 1.4) (drill 0.6) (layers "F.Cu" "B.Cu") (locked yes) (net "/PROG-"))
 (via (at 150.935 118.6624) (size 1.4) (drill 0.6) (layers "F.Cu" "B.Cu") (locked yes) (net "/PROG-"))
 (via (at 162.6529 110.8319) (size 1.4) (drill 0.6) (layers "F.Cu" "B.Cu") (locked yes) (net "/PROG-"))
 (segment (start 161.925 110.104) (end 161.925 97.4278) (width 0.4) (locked yes) (layer "B.Cu") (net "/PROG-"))
 (segment (start 151.8424 119.5698) (end 150.935 118.6624) (width 0.4) (locked yes) (layer "B.Cu") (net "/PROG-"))
 (segment (start 159.8254 122.2935) (end 157.1017 119.5698) (width 0.4) (locked yes) (layer "B.Cu") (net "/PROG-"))
 (segment (start 157.1017 119.5698) (end 151.8424 119.5698) (width 0.4) (locked yes) (layer "B.Cu") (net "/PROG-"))
 (segment (start 162.6529 110.8319) (end 161.925 110.104) (width 0.4) (locked yes) (layer "B.Cu") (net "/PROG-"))
 (segment (start 150.495 109.7196) (end 158.1162 102.0984) (width 0.4) (locked yes) (layer "F.Cu") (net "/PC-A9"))
 (segment (start 147.612 117.8734) (end 150.495 114.9904) (width 0.4) (locked yes) (layer "F.Cu") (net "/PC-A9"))
 (segment (start 150.495 114.9904) (end 150.495 109.7196) (width 0.4) (locked yes) (layer "F.Cu") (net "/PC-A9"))
 (segment (start 165.735 97.79) (end 165.735 117.3755) (width 0.4) (locked yes) (layer "F.Cu") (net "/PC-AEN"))
 (segment (start 163.5407 119.5698) (end 153.7178 119.5698) (width 0.4) (locked yes) (layer "F.Cu") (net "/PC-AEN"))
 (segment (start 165.735 117.3755) (end 163.5407 119.5698) (width 0.4) (locked yes) (layer "F.Cu") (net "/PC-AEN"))
 (segment (start 153.4679 119.8197) (end 141.5629 119.8197) (width 0.4) (locked yes) (layer "F.Cu") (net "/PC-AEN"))
 (segment (start 153.7178 119.5698) (end 153.4679 119.8197) (width 0.4) (locked yes) (layer "F.Cu") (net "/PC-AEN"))
 (segment (start 147.8692 127.4779) (end 167.0281 127.4779) (width 0.4) (locked yes) (layer "F.Cu") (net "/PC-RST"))
 (segment (start 167.0281 127.4779) (end 167.0281 127.478) (width 0.4) (locked yes) (layer "F.Cu") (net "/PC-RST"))
 (via (at 167.0281 127.478) (size 1.4) (drill 0.6) (layers "F.Cu" "B.Cu") (locked yes) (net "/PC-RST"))
 (segment (start 167.0281 127.478) (end 167.0281 131.2008) (width 0.4) (locked yes) (layer "B.Cu") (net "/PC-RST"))
 (segment (start 167.1971 131.3698) (end 167.1971 138.2379) (width 0.4) (locked yes) (layer "B.Cu") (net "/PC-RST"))
 (segment (start 167.0281 131.2008) (end 167.1971 131.3698) (width 0.4) (locked yes) (layer "B.Cu") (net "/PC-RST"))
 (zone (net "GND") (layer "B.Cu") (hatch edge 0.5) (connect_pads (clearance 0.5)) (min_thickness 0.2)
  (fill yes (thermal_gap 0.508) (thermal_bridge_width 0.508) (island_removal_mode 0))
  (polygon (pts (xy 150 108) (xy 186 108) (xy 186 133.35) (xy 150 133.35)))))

